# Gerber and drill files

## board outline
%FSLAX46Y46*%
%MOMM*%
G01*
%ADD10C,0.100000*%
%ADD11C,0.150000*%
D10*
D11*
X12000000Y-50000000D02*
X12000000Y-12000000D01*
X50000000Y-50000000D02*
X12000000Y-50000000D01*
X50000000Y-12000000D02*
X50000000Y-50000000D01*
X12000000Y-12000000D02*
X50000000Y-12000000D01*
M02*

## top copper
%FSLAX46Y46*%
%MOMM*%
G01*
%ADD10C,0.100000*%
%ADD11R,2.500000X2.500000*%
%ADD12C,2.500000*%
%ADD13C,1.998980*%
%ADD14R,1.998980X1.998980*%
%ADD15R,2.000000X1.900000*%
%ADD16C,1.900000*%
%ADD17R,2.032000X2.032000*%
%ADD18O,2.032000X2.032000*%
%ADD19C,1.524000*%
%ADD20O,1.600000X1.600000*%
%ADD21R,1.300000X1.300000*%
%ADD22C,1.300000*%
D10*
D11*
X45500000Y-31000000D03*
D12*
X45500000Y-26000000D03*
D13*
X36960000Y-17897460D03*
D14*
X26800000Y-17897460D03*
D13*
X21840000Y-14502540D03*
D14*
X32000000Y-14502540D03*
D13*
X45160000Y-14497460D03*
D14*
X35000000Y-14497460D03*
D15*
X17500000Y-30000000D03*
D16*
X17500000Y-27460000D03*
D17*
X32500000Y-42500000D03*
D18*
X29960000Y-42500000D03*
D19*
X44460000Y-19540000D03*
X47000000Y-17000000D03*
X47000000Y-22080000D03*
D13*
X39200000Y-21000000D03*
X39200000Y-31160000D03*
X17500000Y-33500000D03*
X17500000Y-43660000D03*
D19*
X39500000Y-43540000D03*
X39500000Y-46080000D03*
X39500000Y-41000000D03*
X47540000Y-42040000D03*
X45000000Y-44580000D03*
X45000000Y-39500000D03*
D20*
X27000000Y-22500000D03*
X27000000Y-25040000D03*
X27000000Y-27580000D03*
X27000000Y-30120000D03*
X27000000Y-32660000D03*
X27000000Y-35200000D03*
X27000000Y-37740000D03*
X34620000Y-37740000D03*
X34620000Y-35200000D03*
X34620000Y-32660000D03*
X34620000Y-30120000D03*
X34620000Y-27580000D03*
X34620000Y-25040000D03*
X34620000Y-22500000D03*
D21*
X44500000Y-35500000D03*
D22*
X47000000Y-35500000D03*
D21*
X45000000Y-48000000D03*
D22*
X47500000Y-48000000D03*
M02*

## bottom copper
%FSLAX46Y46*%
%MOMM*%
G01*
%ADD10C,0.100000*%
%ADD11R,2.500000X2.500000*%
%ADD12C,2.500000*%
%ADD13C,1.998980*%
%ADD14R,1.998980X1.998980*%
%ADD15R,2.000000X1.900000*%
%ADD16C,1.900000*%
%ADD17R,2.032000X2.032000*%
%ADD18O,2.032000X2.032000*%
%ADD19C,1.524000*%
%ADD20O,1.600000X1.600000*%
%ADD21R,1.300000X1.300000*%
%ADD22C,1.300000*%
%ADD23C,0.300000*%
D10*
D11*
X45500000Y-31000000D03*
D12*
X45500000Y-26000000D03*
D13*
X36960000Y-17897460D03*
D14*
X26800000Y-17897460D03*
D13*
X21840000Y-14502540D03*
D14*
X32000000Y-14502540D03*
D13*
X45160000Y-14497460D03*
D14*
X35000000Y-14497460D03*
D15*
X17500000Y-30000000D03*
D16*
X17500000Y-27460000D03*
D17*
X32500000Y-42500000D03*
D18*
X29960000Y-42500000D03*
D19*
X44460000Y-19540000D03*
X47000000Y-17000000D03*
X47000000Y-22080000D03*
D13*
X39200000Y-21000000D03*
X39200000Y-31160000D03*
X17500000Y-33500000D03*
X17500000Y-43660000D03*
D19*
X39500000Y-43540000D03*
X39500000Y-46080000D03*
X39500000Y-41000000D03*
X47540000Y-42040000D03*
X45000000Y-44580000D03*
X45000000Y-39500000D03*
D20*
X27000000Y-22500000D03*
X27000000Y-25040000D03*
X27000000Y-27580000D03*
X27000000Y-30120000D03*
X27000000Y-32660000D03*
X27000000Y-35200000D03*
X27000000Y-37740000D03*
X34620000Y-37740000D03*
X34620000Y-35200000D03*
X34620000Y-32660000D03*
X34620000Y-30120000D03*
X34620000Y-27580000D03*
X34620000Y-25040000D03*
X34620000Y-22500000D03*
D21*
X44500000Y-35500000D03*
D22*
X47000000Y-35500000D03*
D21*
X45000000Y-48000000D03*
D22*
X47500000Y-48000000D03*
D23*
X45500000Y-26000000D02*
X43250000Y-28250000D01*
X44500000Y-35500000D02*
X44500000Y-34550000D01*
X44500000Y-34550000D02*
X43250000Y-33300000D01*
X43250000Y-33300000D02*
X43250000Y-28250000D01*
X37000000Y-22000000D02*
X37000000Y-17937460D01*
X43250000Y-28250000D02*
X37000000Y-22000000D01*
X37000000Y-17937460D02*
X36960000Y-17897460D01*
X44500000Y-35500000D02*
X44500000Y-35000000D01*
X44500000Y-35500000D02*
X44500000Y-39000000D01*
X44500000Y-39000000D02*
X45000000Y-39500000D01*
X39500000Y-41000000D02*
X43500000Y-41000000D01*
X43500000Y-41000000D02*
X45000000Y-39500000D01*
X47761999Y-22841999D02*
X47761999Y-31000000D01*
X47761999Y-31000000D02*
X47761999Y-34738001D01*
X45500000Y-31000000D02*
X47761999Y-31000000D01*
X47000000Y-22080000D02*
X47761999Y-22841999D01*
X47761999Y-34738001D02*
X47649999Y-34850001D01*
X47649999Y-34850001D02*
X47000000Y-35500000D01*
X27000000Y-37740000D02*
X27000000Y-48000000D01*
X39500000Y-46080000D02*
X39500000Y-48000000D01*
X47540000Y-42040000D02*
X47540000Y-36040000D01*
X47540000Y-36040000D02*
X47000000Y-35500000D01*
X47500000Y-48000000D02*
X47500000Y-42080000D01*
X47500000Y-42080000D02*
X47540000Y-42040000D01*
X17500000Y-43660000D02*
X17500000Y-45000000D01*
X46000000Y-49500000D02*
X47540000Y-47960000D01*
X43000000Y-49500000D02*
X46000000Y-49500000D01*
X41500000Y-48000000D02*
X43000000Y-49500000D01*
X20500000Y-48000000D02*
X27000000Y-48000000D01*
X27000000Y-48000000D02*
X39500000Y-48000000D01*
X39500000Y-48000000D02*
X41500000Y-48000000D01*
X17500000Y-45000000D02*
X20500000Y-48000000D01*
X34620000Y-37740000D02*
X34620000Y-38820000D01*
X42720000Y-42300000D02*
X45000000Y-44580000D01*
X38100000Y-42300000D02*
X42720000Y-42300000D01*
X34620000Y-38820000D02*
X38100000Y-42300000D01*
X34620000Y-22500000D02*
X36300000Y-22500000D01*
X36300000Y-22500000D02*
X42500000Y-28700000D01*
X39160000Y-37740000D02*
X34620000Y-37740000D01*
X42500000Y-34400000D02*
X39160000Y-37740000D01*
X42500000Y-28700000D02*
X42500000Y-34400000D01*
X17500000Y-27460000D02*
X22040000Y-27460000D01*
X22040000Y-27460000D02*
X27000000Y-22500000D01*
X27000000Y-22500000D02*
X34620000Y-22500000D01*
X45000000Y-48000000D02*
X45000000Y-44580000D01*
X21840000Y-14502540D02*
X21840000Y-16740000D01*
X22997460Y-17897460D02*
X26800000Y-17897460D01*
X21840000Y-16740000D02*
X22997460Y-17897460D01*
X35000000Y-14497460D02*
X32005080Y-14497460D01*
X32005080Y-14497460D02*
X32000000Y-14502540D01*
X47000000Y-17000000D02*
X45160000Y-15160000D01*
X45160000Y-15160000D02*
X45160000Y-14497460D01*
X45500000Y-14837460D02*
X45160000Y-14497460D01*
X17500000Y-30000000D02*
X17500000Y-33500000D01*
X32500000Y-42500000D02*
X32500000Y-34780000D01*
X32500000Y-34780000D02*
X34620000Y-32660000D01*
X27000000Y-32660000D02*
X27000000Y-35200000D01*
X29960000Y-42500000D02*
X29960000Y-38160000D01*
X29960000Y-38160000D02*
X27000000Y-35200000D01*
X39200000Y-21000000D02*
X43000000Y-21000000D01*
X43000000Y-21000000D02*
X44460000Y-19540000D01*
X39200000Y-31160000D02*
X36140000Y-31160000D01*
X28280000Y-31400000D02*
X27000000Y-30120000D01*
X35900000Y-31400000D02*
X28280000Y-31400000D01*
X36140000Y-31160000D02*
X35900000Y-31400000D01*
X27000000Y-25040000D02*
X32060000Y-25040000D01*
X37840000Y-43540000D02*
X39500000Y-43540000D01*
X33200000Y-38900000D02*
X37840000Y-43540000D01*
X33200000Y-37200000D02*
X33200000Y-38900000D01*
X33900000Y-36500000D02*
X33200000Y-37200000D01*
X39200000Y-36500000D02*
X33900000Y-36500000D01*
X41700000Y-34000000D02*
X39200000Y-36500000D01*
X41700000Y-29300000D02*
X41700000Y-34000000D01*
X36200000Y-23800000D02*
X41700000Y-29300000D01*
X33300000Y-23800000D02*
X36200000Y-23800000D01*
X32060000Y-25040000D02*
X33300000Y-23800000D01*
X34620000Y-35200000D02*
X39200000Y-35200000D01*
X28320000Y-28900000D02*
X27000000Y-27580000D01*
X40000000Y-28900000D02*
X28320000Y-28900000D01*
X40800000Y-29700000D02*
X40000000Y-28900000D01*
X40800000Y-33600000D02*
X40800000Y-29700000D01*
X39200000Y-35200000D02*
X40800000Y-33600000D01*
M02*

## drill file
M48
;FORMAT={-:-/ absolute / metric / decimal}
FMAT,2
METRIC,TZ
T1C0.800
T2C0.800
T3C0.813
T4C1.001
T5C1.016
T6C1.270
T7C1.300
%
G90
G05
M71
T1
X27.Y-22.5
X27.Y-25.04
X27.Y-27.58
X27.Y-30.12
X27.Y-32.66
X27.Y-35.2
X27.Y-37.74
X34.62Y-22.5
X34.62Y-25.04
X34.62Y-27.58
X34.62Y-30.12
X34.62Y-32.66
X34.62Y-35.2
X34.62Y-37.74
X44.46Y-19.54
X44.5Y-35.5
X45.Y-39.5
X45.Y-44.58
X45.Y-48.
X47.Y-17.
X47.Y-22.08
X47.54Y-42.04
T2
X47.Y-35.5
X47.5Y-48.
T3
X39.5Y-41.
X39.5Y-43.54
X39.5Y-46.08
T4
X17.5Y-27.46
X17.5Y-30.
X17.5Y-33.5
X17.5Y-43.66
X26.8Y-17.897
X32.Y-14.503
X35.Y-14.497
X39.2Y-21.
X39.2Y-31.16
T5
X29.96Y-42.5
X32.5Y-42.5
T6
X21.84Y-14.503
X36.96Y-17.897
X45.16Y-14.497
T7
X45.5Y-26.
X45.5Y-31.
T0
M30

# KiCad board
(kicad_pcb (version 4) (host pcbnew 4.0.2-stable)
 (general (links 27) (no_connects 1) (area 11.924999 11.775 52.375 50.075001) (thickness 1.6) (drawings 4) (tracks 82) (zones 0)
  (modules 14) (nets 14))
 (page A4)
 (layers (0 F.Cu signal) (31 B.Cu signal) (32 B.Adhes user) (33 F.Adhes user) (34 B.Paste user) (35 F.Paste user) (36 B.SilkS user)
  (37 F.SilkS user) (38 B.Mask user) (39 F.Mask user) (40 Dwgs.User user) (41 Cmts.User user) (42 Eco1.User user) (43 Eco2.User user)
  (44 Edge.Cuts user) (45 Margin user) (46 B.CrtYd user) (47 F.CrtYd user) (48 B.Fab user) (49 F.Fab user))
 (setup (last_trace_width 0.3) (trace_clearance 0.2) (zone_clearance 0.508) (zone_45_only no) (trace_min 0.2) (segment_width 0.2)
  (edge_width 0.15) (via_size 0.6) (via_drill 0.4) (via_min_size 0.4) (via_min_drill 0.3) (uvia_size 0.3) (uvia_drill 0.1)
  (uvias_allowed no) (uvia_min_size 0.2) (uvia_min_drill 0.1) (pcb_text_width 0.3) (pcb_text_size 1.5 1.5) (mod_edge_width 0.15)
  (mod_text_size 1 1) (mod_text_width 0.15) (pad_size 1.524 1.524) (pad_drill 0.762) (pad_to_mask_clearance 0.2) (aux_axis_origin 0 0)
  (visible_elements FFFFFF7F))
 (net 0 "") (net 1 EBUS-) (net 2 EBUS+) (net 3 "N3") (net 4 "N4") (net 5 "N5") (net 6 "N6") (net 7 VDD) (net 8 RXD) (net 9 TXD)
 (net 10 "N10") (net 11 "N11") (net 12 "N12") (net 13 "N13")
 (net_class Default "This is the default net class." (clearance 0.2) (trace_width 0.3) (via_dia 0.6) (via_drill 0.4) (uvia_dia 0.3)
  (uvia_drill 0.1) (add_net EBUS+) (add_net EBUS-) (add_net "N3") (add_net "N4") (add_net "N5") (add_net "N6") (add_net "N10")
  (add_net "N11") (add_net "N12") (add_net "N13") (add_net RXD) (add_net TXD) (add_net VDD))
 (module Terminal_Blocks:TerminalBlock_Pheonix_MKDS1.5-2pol (layer F.Cu) (at 45.5 31 90)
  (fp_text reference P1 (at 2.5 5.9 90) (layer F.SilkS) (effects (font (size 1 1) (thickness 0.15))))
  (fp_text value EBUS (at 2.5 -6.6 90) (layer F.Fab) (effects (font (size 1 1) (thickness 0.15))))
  (pad 1 thru_hole rect (at 0 0 90) (size 2.5 2.5) (drill 1.3) (layers *.Cu *.Mask F.SilkS) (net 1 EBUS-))
  (pad 2 thru_hole circle (at 5 0 90) (size 2.5 2.5) (drill 1.3) (layers *.Cu *.Mask F.SilkS) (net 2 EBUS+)))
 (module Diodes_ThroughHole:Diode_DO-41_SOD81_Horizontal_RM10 (layer F.Cu) (at 26.8 17.9)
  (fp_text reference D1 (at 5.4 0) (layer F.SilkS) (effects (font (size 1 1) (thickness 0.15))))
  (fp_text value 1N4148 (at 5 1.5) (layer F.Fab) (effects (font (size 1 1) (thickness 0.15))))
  (pad 2 thru_hole circle (at 10.16 -0.00254 180) (size 1.99898 1.99898) (drill 1.27) (layers *.Cu *.Mask F.SilkS) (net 2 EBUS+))
  (pad 1 thru_hole rect (at 0 -0.00254 180) (size 1.99898 1.99898) (drill 1.00076) (layers *.Cu *.Mask F.SilkS) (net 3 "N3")))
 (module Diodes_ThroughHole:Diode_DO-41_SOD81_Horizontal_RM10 (layer F.Cu) (at 32 14.5 180)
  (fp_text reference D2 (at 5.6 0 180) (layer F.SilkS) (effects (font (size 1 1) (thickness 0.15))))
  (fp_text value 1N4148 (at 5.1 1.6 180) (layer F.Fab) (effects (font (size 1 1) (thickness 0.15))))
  (pad 2 thru_hole circle (at 10.16 -0.00254) (size 1.99898 1.99898) (drill 1.27) (layers *.Cu *.Mask F.SilkS) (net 3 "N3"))
  (pad 1 thru_hole rect (at 0 -0.00254) (size 1.99898 1.99898) (drill 1.00076) (layers *.Cu *.Mask F.SilkS) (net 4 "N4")))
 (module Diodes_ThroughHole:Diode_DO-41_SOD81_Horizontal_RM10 (layer F.Cu) (at 35 14.5)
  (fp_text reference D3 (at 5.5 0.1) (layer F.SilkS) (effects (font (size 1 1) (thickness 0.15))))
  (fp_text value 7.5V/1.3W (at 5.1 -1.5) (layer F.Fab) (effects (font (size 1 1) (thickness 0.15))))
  (pad 2 thru_hole circle (at 10.16 -0.00254 180) (size 1.99898 1.99898) (drill 1.27) (layers *.Cu *.Mask F.SilkS) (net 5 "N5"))
  (pad 1 thru_hole rect (at 0 -0.00254 180) (size 1.99898 1.99898) (drill 1.00076) (layers *.Cu *.Mask F.SilkS) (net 4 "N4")))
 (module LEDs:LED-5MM (layer F.Cu) (at 17.5 30 90)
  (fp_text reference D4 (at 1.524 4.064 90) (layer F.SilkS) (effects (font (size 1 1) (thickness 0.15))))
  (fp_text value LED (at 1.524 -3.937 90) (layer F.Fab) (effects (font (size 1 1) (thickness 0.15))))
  (pad 1 thru_hole rect (at 0 0 180) (size 2 1.9) (drill 1.00076) (layers *.Cu *.Mask F.SilkS) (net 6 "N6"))
  (pad 2 thru_hole circle (at 2.54 0 90) (size 1.9 1.9) (drill 1.00076) (layers *.Cu *.Mask F.SilkS) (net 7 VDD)))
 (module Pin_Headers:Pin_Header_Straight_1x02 (layer F.Cu) (at 32.5 42.5 270)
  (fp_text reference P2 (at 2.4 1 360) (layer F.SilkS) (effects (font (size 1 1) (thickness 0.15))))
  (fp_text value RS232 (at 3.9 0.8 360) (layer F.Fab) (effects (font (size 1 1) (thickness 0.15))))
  (pad 1 thru_hole rect (at 0 0 270) (size 2.032 2.032) (drill 1.016) (layers *.Cu *.Mask F.SilkS) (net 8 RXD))
  (pad 2 thru_hole oval (at 0 2.54 270) (size 2.032 2.032) (drill 1.016) (layers *.Cu *.Mask F.SilkS) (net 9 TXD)))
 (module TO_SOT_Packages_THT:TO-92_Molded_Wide (layer F.Cu) (at 47 22.08 90)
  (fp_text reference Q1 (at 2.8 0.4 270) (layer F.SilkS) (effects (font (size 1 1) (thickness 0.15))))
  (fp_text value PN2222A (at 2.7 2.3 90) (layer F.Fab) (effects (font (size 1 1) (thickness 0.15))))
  (pad 2 thru_hole circle (at 2.54 -2.54 180) (size 1.524 1.524) (drill 0.8) (layers *.Cu *.Mask F.SilkS) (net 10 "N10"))
  (pad 3 thru_hole circle (at 5.08 0 180) (size 1.524 1.524) (drill 0.8) (layers *.Cu *.Mask F.SilkS) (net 5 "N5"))
  (pad 1 thru_hole circle (at 0 0 180) (size 1.524 1.524) (drill 0.8) (layers *.Cu *.Mask F.SilkS) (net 1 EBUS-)))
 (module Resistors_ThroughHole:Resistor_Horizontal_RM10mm (layer F.Cu) (at 39.2 21 270)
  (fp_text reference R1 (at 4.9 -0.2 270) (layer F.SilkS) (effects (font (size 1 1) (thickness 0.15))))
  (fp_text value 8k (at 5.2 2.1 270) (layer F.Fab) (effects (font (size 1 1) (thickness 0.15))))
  (pad 1 thru_hole circle (at 0 0 270) (size 1.99898 1.99898) (drill 1.00076) (layers *.Cu *.SilkS *.Mask) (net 10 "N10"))
  (pad 2 thru_hole circle (at 10.16 0 270) (size 1.99898 1.99898) (drill 1.00076) (layers *.Cu *.SilkS *.Mask) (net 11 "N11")))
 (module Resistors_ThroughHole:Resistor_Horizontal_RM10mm (layer F.Cu) (at 17.5 33.5 270)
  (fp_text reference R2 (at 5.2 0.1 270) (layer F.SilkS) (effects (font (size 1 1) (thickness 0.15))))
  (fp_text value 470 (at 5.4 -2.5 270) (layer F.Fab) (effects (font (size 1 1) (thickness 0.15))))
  (pad 1 thru_hole circle (at 0 0 270) (size 1.99898 1.99898) (drill 1.00076) (layers *.Cu *.SilkS *.Mask) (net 6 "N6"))
  (pad 2 thru_hole circle (at 10.16 0 270) (size 1.99898 1.99898) (drill 1.00076) (layers *.Cu *.SilkS *.Mask) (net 1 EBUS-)))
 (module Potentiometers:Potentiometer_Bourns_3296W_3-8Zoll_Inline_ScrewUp (layer F.Cu) (at 39.5 41 180)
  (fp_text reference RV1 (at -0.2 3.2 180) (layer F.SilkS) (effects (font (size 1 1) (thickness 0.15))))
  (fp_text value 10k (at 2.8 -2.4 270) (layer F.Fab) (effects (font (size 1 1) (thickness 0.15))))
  (pad 2 thru_hole circle (at 0 -2.54 180) (size 1.524 1.524) (drill 0.8128) (layers *.Cu *.Mask F.SilkS) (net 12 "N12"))
  (pad 3 thru_hole circle (at 0 -5.08 180) (size 1.524 1.524) (drill 0.8128) (layers *.Cu *.Mask F.SilkS) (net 1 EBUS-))
  (pad 1 thru_hole circle (at 0 0 180) (size 1.524 1.524) (drill 0.8128) (layers *.Cu *.Mask F.SilkS) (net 2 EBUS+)))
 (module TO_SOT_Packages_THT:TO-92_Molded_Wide (layer F.Cu) (at 45 39.5 270)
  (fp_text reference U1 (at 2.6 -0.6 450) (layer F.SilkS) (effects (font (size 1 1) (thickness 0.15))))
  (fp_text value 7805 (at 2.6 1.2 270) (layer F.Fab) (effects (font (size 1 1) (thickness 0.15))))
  (pad 2 thru_hole circle (at 2.54 -2.54) (size 1.524 1.524) (drill 0.8) (layers *.Cu *.Mask F.SilkS) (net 1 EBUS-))
  (pad 3 thru_hole circle (at 5.08 0) (size 1.524 1.524) (drill 0.8) (layers *.Cu *.Mask F.SilkS) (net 7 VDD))
  (pad 1 thru_hole circle (at 0 0) (size 1.524 1.524) (drill 0.8) (layers *.Cu *.Mask F.SilkS) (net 2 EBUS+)))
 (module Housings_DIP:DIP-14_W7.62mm (layer F.Cu) (at 27 22.5)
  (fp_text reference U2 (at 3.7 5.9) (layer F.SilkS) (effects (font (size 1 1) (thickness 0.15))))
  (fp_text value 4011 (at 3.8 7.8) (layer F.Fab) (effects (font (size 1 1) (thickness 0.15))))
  (pad 1 thru_hole oval (at 0 0) (size 1.6 1.6) (drill 0.8) (layers *.Cu *.Mask F.SilkS) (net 7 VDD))
  (pad 2 thru_hole oval (at 0 2.54) (size 1.6 1.6) (drill 0.8) (layers *.Cu *.Mask F.SilkS) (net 12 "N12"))
  (pad 3 thru_hole oval (at 0 5.08) (size 1.6 1.6) (drill 0.8) (layers *.Cu *.Mask F.SilkS) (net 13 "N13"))
  (pad 4 thru_hole oval (at 0 7.62) (size 1.6 1.6) (drill 0.8) (layers *.Cu *.Mask F.SilkS) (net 11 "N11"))
  (pad 5 thru_hole oval (at 0 10.16) (size 1.6 1.6) (drill 0.8) (layers *.Cu *.Mask F.SilkS) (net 9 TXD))
  (pad 6 thru_hole oval (at 0 12.7) (size 1.6 1.6) (drill 0.8) (layers *.Cu *.Mask F.SilkS) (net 9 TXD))
  (pad 7 thru_hole oval (at 0 15.24) (size 1.6 1.6) (drill 0.8) (layers *.Cu *.Mask F.SilkS) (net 1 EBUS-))
  (pad 8 thru_hole oval (at 7.62 15.24) (size 1.6 1.6) (drill 0.8) (layers *.Cu *.Mask F.SilkS) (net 7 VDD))
  (pad 9 thru_hole oval (at 7.62 12.7) (size 1.6 1.6) (drill 0.8) (layers *.Cu *.Mask F.SilkS) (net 13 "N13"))
  (pad 10 thru_hole oval (at 7.62 10.16) (size 1.6 1.6) (drill 0.8) (layers *.Cu *.Mask F.SilkS) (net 8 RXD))
  (pad 11 thru_hole oval (at 7.62 7.62) (size 1.6 1.6) (drill 0.8) (layers *.Cu *.Mask F.SilkS))
  (pad 12 thru_hole oval (at 7.62 5.08) (size 1.6 1.6) (drill 0.8) (layers *.Cu *.Mask F.SilkS))
  (pad 13 thru_hole oval (at 7.62 2.54) (size 1.6 1.6) (drill 0.8) (layers *.Cu *.Mask F.SilkS))
  (pad 14 thru_hole oval (at 7.62 0) (size 1.6 1.6) (drill 0.8) (layers *.Cu *.Mask F.SilkS) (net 7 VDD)))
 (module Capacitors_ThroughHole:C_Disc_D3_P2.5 (layer F.Cu) (at 44.5 35.5)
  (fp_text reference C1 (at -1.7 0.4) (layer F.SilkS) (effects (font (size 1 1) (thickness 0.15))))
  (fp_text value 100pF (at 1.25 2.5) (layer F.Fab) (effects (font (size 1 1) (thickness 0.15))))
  (pad 1 thru_hole rect (at 0 0) (size 1.3 1.3) (drill 0.8) (layers *.Cu *.Mask F.SilkS) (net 2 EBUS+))
  (pad 2 thru_hole circle (at 2.5 0) (size 1.3 1.3) (drill 0.8001) (layers *.Cu *.Mask F.SilkS) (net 1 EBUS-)))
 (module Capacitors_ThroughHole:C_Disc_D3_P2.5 (layer F.Cu) (at 45 48)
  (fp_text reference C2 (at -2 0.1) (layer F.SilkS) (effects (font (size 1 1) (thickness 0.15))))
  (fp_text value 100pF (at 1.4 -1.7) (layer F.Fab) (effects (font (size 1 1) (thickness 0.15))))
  (pad 1 thru_hole rect (at 0 0) (size 1.3 1.3) (drill 0.8) (layers *.Cu *.Mask F.SilkS) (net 7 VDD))
  (pad 2 thru_hole circle (at 2.5 0) (size 1.3 1.3) (drill 0.8001) (layers *.Cu *.Mask F.SilkS) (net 1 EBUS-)))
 (gr_line (start 12 50) (end 12 12) (angle 90) (layer Edge.Cuts) (width 0.15))
 (gr_line (start 50 50) (end 12 50) (angle 90) (layer Edge.Cuts) (width 0.15))
 (gr_line (start 50 12) (end 50 50) (angle 90) (layer Edge.Cuts) (width 0.15))
 (gr_line (start 12 12) (end 50 12) (angle 90) (layer Edge.Cuts) (width 0.15))
 (segment (start 45.5 26) (end 43.25 28.25) (width 0.3) (layer B.Cu) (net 2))
 (segment (start 44.5 35.5) (end 44.5 34.55) (width 0.3) (layer B.Cu) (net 2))
 (segment (start 44.5 34.55) (end 43.25 33.3) (width 0.3) (layer B.Cu) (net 2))
 (segment (start 43.25 33.3) (end 43.25 28.25) (width 0.3) (layer B.Cu) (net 2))
 (segment (start 37 22) (end 37 17.93746) (width 0.3) (layer B.Cu) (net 2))
 (segment (start 43.25 28.25) (end 37 22) (width 0.3) (layer B.Cu) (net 2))
 (segment (start 37 17.93746) (end 36.96 17.89746) (width 0.3) (layer B.Cu) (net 2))
 (segment (start 44.5 35.5) (end 44.5 35) (width 0.3) (layer B.Cu) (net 2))
 (segment (start 44.5 35.5) (end 44.5 39) (width 0.3) (layer B.Cu) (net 2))
 (segment (start 44.5 39) (end 45 39.5) (width 0.3) (layer B.Cu) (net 2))
 (segment (start 39.5 41) (end 43.5 41) (width 0.3) (layer B.Cu) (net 2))
 (segment (start 43.5 41) (end 45 39.5) (width 0.3) (layer B.Cu) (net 2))
 (segment (start 47.761999 22.841999) (end 47.761999 31) (width 0.3) (layer B.Cu) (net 1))
 (segment (start 47.761999 31) (end 47.761999 34.738001) (width 0.3) (layer B.Cu) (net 1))
 (segment (start 45.5 31) (end 47.761999 31) (width 0.3) (layer B.Cu) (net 1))
 (segment (start 47 22.08) (end 47.761999 22.841999) (width 0.3) (layer B.Cu) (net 1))
 (segment (start 47.761999 34.738001) (end 47.649999 34.850001) (width 0.3) (layer B.Cu) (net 1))
 (segment (start 47.649999 34.850001) (end 47 35.5) (width 0.3) (layer B.Cu) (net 1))
 (segment (start 27 37.74) (end 27 48) (width 0.3) (layer B.Cu) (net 1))
 (segment (start 39.5 46.08) (end 39.5 48) (width 0.3) (layer B.Cu) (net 1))
 (segment (start 47.54 42.04) (end 47.54 36.04) (width 0.3) (layer B.Cu) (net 1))
 (segment (start 47.54 36.04) (end 47 35.5) (width 0.3) (layer B.Cu) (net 1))
 (segment (start 47.5 48) (end 47.5 42.08) (width 0.3) (layer B.Cu) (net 1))
 (segment (start 47.5 42.08) (end 47.54 42.04) (width 0.3) (layer B.Cu) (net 1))
 (segment (start 17.5 43.66) (end 17.5 45) (width 0.3) (layer B.Cu) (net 1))
 (segment (start 46 49.5) (end 47.54 47.96) (width 0.3) (layer B.Cu) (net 1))
 (segment (start 43 49.5) (end 46 49.5) (width 0.3) (layer B.Cu) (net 1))
 (segment (start 41.5 48) (end 43 49.5) (width 0.3) (layer B.Cu) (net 1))
 (segment (start 20.5 48) (end 27 48) (width 0.3) (layer B.Cu) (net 1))
 (segment (start 27 48) (end 39.5 48) (width 0.3) (layer B.Cu) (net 1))
 (segment (start 39.5 48) (end 41.5 48) (width 0.3) (layer B.Cu) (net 1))
 (segment (start 17.5 45) (end 20.5 48) (width 0.3) (layer B.Cu) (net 1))
 (segment (start 34.62 37.74) (end 34.62 38.82) (width 0.3) (layer B.Cu) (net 7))
 (segment (start 42.72 42.3) (end 45 44.58) (width 0.3) (layer B.Cu) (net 7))
 (segment (start 38.1 42.3) (end 42.72 42.3) (width 0.3) (layer B.Cu) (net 7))
 (segment (start 34.62 38.82) (end 38.1 42.3) (width 0.3) (layer B.Cu) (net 7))
 (segment (start 34.62 22.5) (end 36.3 22.5) (width 0.3) (layer B.Cu) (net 7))
 (segment (start 36.3 22.5) (end 42.5 28.7) (width 0.3) (layer B.Cu) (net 7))
 (segment (start 39.16 37.74) (end 34.62 37.74) (width 0.3) (layer B.Cu) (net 7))
 (segment (start 42.5 34.4) (end 39.16 37.74) (width 0.3) (layer B.Cu) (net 7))
 (segment (start 42.5 28.7) (end 42.5 34.4) (width 0.3) (layer B.Cu) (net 7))
 (segment (start 17.5 27.46) (end 22.04 27.46) (width 0.3) (layer B.Cu) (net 7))
 (segment (start 22.04 27.46) (end 27 22.5) (width 0.3) (layer B.Cu) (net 7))
 (segment (start 27 22.5) (end 34.62 22.5) (width 0.3) (layer B.Cu) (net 7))
 (segment (start 45 48) (end 45 44.58) (width 0.3) (layer B.Cu) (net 7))
 (segment (start 21.84 14.50254) (end 21.84 16.74) (width 0.3) (layer B.Cu) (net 3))
 (segment (start 22.99746 17.89746) (end 26.8 17.89746) (width 0.3) (layer B.Cu) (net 3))
 (segment (start 21.84 16.74) (end 22.99746 17.89746) (width 0.3) (layer B.Cu) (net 3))
 (segment (start 35 14.49746) (end 32.00508 14.49746) (width 0.3) (layer B.Cu) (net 4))
 (segment (start 32.00508 14.49746) (end 32 14.50254) (width 0.3) (layer B.Cu) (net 4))
 (segment (start 47 17) (end 45.16 15.16) (width 0.3) (layer B.Cu) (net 5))
 (segment (start 45.16 15.16) (end 45.16 14.49746) (width 0.3) (layer B.Cu) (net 5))
 (segment (start 45.5 14.83746) (end 45.16 14.49746) (width 0.3) (layer B.Cu) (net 5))
 (segment (start 17.5 30) (end 17.5 33.5) (width 0.3) (layer B.Cu) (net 6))
 (segment (start 32.5 42.5) (end 32.5 34.78) (width 0.3) (layer B.Cu) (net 8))
 (segment (start 32.5 34.78) (end 34.62 32.66) (width 0.3) (layer B.Cu) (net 8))
 (segment (start 27 32.66) (end 27 35.2) (width 0.3) (layer B.Cu) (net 9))
 (segment (start 29.96 42.5) (end 29.96 38.16) (width 0.3) (layer B.Cu) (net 9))
 (segment (start 29.96 38.16) (end 27 35.2) (width 0.3) (layer B.Cu) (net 9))
 (segment (start 39.2 21) (end 43 21) (width 0.3) (layer B.Cu) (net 10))
 (segment (start 43 21) (end 44.46 19.54) (width 0.3) (layer B.Cu) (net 10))
 (segment (start 39.2 31.16) (end 36.14 31.16) (width 0.3) (layer B.Cu) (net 11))
 (segment (start 28.28 31.4) (end 27 30.12) (width 0.3) (layer B.Cu) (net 11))
 (segment (start 35.9 31.4) (end 28.28 31.4) (width 0.3) (layer B.Cu) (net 11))
 (segment (start 36.14 31.16) (end 35.9 31.4) (width 0.3) (layer B.Cu) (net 11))
 (segment (start 27 25.04) (end 32.06 25.04) (width 0.3) (layer B.Cu) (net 12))
 (segment (start 37.84 43.54) (end 39.5 43.54) (width 0.3) (layer B.Cu) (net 12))
 (segment (start 33.2 38.9) (end 37.84 43.54) (width 0.3) (layer B.Cu) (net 12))
 (segment (start 33.2 37.2) (end 33.2 38.9) (width 0.3) (layer B.Cu) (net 12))
 (segment (start 33.9 36.5) (end 33.2 37.2) (width 0.3) (layer B.Cu) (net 12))
 (segment (start 39.2 36.5) (end 33.9 36.5) (width 0.3) (layer B.Cu) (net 12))
 (segment (start 41.7 34) (end 39.2 36.5) (width 0.3) (layer B.Cu) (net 12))
 (segment (start 41.7 29.3) (end 41.7 34) (width 0.3) (layer B.Cu) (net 12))
 (segment (start 36.2 23.8) (end 41.7 29.3) (width 0.3) (layer B.Cu) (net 12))
 (segment (start 33.3 23.8) (end 36.2 23.8) (width 0.3) (layer B.Cu) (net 12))
 (segment (start 32.06 25.04) (end 33.3 23.8) (width 0.3) (layer B.Cu) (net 12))
 (segment (start 34.62 35.2) (end 39.2 35.2) (width 0.3) (layer B.Cu) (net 13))
 (segment (start 28.32 28.9) (end 27 27.58) (width 0.3) (layer B.Cu) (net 13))
 (segment (start 40 28.9) (end 28.32 28.9) (width 0.3) (layer B.Cu) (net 13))
 (segment (start 40.8 29.7) (end 40 28.9) (width 0.3) (layer B.Cu) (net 13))
 (segment (start 40.8 33.6) (end 40.8 29.7) (width 0.3) (layer B.Cu) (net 13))
 (segment (start 39.2 35.2) (end 40.8 33.6) (width 0.3) (layer B.Cu) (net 13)))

